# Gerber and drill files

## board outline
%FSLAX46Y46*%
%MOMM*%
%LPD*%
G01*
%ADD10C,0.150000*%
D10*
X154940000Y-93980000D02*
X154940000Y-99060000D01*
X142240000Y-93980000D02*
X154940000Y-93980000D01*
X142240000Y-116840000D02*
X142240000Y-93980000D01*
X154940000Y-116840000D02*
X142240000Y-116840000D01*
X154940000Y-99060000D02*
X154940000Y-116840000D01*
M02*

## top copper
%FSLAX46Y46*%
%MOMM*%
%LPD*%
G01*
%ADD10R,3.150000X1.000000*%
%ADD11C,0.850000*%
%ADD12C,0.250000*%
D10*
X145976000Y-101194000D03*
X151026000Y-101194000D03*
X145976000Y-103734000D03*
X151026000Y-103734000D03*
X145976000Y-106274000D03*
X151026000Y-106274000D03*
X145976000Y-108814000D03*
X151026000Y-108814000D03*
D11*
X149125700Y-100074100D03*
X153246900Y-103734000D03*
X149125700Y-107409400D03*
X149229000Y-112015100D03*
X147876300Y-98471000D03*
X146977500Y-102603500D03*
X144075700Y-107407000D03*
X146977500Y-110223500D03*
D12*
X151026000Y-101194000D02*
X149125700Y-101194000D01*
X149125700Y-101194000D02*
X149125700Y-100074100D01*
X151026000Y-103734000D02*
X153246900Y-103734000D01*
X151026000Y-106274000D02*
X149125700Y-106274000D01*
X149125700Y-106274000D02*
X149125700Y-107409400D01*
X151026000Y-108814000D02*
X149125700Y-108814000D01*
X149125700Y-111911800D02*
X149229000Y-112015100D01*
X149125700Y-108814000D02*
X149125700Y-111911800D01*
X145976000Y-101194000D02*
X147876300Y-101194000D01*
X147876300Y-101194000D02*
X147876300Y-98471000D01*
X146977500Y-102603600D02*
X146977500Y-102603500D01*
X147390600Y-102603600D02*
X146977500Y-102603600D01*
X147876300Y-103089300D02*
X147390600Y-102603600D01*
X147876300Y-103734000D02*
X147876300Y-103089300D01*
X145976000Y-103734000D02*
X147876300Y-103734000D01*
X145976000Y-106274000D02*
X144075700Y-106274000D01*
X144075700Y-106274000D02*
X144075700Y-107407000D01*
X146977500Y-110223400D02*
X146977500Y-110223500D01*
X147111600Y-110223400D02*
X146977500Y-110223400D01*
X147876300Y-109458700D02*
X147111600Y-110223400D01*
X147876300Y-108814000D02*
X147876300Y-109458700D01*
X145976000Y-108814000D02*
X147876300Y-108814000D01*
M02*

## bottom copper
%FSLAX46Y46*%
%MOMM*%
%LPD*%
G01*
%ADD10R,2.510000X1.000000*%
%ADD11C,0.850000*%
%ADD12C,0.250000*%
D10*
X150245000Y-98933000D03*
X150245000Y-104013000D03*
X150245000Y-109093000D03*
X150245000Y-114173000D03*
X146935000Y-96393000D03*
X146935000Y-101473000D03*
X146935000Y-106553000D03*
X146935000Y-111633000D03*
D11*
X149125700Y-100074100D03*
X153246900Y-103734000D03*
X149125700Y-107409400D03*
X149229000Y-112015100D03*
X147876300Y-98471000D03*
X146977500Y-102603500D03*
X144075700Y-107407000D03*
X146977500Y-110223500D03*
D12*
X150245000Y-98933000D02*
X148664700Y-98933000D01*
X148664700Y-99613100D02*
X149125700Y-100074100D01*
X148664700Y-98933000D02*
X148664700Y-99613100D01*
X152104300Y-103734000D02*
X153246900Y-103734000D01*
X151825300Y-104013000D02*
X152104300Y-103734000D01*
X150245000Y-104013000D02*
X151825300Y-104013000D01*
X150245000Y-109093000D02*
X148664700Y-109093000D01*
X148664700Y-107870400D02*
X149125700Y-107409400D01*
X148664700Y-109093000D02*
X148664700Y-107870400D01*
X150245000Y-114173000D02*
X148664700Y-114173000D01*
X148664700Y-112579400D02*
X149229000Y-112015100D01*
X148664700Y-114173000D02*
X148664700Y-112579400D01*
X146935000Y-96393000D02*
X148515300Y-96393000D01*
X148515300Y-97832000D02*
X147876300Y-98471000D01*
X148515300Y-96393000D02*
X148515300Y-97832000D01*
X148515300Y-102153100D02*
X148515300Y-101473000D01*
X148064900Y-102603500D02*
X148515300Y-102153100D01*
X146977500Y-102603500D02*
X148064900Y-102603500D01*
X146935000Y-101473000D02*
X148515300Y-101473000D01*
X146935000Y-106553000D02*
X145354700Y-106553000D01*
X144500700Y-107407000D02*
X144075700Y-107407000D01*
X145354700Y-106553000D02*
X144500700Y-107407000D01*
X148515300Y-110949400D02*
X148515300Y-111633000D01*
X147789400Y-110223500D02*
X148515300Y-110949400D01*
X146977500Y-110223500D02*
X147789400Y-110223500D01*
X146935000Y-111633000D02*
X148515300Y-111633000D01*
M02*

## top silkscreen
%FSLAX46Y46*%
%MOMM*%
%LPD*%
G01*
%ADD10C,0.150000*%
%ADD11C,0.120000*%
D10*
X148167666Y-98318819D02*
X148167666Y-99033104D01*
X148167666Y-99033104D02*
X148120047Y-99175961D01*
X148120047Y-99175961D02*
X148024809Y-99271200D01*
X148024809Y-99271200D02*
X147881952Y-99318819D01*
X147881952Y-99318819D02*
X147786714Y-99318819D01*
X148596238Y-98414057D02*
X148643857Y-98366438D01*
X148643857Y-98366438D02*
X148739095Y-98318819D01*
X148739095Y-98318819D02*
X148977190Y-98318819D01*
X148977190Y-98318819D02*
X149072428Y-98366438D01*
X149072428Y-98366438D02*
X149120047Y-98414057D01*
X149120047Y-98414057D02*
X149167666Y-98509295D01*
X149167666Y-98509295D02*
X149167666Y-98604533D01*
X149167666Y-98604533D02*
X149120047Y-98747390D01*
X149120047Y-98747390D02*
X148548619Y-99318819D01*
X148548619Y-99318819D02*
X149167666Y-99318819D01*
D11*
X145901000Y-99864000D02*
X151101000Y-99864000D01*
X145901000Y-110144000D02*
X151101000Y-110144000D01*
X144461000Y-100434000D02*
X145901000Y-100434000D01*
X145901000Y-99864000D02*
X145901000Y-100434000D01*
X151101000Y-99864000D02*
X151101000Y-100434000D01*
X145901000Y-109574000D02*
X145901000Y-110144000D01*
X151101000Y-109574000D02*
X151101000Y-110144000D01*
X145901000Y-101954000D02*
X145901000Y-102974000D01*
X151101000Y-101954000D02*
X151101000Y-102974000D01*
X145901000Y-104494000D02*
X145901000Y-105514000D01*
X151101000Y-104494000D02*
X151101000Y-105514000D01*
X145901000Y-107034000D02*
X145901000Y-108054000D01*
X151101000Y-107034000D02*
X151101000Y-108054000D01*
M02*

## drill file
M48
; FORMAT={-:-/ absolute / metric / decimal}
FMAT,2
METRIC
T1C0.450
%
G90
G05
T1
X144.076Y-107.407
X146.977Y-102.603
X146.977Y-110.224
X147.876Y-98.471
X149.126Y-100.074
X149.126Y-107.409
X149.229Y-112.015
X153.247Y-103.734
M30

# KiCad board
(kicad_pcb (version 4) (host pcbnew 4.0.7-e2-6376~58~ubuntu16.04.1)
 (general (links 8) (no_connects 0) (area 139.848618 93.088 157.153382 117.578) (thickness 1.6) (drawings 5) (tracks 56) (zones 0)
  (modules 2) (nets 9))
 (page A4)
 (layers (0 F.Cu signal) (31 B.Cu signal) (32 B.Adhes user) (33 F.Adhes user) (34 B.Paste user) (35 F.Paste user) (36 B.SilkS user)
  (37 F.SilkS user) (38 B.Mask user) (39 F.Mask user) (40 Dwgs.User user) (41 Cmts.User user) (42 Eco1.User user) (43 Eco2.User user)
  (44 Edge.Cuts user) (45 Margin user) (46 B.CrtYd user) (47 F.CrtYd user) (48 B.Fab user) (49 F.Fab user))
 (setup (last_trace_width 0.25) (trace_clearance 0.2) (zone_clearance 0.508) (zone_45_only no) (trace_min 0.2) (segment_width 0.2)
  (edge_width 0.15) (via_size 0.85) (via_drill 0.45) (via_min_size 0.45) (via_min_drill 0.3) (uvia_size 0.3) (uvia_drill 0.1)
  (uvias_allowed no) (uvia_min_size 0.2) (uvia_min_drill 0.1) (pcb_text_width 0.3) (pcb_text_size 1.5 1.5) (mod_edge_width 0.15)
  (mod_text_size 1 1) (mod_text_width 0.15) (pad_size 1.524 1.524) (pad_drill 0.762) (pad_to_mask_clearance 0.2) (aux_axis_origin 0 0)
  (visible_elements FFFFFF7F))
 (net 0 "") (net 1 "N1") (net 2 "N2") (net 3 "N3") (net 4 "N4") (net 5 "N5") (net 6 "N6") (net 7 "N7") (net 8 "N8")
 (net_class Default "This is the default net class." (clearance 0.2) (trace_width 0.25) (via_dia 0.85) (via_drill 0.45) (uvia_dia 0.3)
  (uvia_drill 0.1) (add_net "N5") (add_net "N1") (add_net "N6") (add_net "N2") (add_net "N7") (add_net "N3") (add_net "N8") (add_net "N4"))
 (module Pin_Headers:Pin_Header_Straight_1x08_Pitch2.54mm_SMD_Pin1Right (layer B.Cu) (at 148.59 105.283 180)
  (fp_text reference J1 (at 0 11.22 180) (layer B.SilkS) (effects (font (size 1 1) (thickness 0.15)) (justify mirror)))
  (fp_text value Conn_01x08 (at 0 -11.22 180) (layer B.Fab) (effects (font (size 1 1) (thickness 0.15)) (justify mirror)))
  (pad 2 smd rect (at -1.655 6.35 180) (size 2.51 1) (layers B.Cu B.Paste B.Mask) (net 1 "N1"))
  (pad 4 smd rect (at -1.655 1.27 180) (size 2.51 1) (layers B.Cu B.Paste B.Mask) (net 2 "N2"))
  (pad 6 smd rect (at -1.655 -3.81 180) (size 2.51 1) (layers B.Cu B.Paste B.Mask) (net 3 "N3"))
  (pad 8 smd rect (at -1.655 -8.89 180) (size 2.51 1) (layers B.Cu B.Paste B.Mask) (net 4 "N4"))
  (pad 1 smd rect (at 1.655 8.89 180) (size 2.51 1) (layers B.Cu B.Paste B.Mask) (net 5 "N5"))
  (pad 3 smd rect (at 1.655 3.81 180) (size 2.51 1) (layers B.Cu B.Paste B.Mask) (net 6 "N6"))
  (pad 5 smd rect (at 1.655 -1.27 180) (size 2.51 1) (layers B.Cu B.Paste B.Mask) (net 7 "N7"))
  (pad 7 smd rect (at 1.655 -6.35 180) (size 2.51 1) (layers B.Cu B.Paste B.Mask) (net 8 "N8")))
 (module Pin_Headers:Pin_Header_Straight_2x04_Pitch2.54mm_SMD (layer F.Cu) (at 148.501 105.004)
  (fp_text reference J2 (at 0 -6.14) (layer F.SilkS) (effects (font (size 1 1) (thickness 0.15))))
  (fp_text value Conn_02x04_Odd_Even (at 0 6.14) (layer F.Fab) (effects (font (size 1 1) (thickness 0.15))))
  (fp_line (start -2.6 -5.14) (end 2.6 -5.14) (layer F.SilkS) (width 0.12))
  (fp_line (start -2.6 5.14) (end 2.6 5.14) (layer F.SilkS) (width 0.12))
  (fp_line (start -4.04 -4.57) (end -2.6 -4.57) (layer F.SilkS) (width 0.12))
  (fp_line (start -2.6 -5.14) (end -2.6 -4.57) (layer F.SilkS) (width 0.12))
  (fp_line (start 2.6 -5.14) (end 2.6 -4.57) (layer F.SilkS) (width 0.12))
  (fp_line (start -2.6 4.57) (end -2.6 5.14) (layer F.SilkS) (width 0.12))
  (fp_line (start 2.6 4.57) (end 2.6 5.14) (layer F.SilkS) (width 0.12))
  (fp_line (start -2.6 -3.05) (end -2.6 -2.03) (layer F.SilkS) (width 0.12))
  (fp_line (start 2.6 -3.05) (end 2.6 -2.03) (layer F.SilkS) (width 0.12))
  (fp_line (start -2.6 -0.51) (end -2.6 0.51) (layer F.SilkS) (width 0.12))
  (fp_line (start 2.6 -0.51) (end 2.6 0.51) (layer F.SilkS) (width 0.12))
  (fp_line (start -2.6 2.03) (end -2.6 3.05) (layer F.SilkS) (width 0.12))
  (fp_line (start 2.6 2.03) (end 2.6 3.05) (layer F.SilkS) (width 0.12))
  (pad 1 smd rect (at -2.525 -3.81) (size 3.15 1) (layers F.Cu F.Paste F.Mask) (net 5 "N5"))
  (pad 2 smd rect (at 2.525 -3.81) (size 3.15 1) (layers F.Cu F.Paste F.Mask) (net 1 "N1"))
  (pad 3 smd rect (at -2.525 -1.27) (size 3.15 1) (layers F.Cu F.Paste F.Mask) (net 6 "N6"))
  (pad 4 smd rect (at 2.525 -1.27) (size 3.15 1) (layers F.Cu F.Paste F.Mask) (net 2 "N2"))
  (pad 5 smd rect (at -2.525 1.27) (size 3.15 1) (layers F.Cu F.Paste F.Mask) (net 7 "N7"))
  (pad 6 smd rect (at 2.525 1.27) (size 3.15 1) (layers F.Cu F.Paste F.Mask) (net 3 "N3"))
  (pad 7 smd rect (at -2.525 3.81) (size 3.15 1) (layers F.Cu F.Paste F.Mask) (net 8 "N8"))
  (pad 8 smd rect (at 2.525 3.81) (size 3.15 1) (layers F.Cu F.Paste F.Mask) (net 4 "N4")))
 (gr_line (start 154.94 93.98) (end 154.94 99.06) (layer Edge.Cuts) (width 0.15))
 (gr_line (start 142.24 93.98) (end 154.94 93.98) (layer Edge.Cuts) (width 0.15))
 (gr_line (start 142.24 116.84) (end 142.24 93.98) (layer Edge.Cuts) (width 0.15))
 (gr_line (start 154.94 116.84) (end 142.24 116.84) (layer Edge.Cuts) (width 0.15))
 (gr_line (start 154.94 99.06) (end 154.94 116.84) (layer Edge.Cuts) (width 0.15))
 (via (at 149.1257 100.0741) (size 0.85) (layers F.Cu B.Cu) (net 1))
 (segment (start 151.026 101.194) (end 149.1257 101.194) (width 0.25) (layer F.Cu) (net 1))
 (segment (start 150.245 98.933) (end 148.6647 98.933) (width 0.25) (layer B.Cu) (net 1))
 (segment (start 148.6647 99.6131) (end 149.1257 100.0741) (width 0.25) (layer B.Cu) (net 1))
 (segment (start 148.6647 98.933) (end 148.6647 99.6131) (width 0.25) (layer B.Cu) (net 1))
 (segment (start 149.1257 101.194) (end 149.1257 100.0741) (width 0.25) (layer F.Cu) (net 1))
 (via (at 153.2469 103.734) (size 0.85) (layers F.Cu B.Cu) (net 2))
 (segment (start 152.1043 103.734) (end 153.2469 103.734) (width 0.25) (layer B.Cu) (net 2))
 (segment (start 151.8253 104.013) (end 152.1043 103.734) (width 0.25) (layer B.Cu) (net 2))
 (segment (start 151.026 103.734) (end 153.2469 103.734) (width 0.25) (layer F.Cu) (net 2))
 (segment (start 150.245 104.013) (end 151.8253 104.013) (width 0.25) (layer B.Cu) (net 2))
 (via (at 149.1257 107.4094) (size 0.85) (layers F.Cu B.Cu) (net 3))
 (segment (start 151.026 106.274) (end 149.1257 106.274) (width 0.25) (layer F.Cu) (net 3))
 (segment (start 150.245 109.093) (end 148.6647 109.093) (width 0.25) (layer B.Cu) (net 3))
 (segment (start 148.6647 107.8704) (end 149.1257 107.4094) (width 0.25) (layer B.Cu) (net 3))
 (segment (start 148.6647 109.093) (end 148.6647 107.8704) (width 0.25) (layer B.Cu) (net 3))
 (segment (start 149.1257 106.274) (end 149.1257 107.4094) (width 0.25) (layer F.Cu) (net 3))
 (via (at 149.229 112.0151) (size 0.85) (layers F.Cu B.Cu) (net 4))
 (segment (start 150.245 114.173) (end 148.6647 114.173) (width 0.25) (layer B.Cu) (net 4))
 (segment (start 151.026 108.814) (end 149.1257 108.814) (width 0.25) (layer F.Cu) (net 4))
 (segment (start 148.6647 112.5794) (end 149.229 112.0151) (width 0.25) (layer B.Cu) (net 4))
 (segment (start 148.6647 114.173) (end 148.6647 112.5794) (width 0.25) (layer B.Cu) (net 4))
 (segment (start 149.1257 111.9118) (end 149.229 112.0151) (width 0.25) (layer F.Cu) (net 4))
 (segment (start 149.1257 108.814) (end 149.1257 111.9118) (width 0.25) (layer F.Cu) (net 4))
 (via (at 147.8763 98.471) (size 0.85) (layers F.Cu B.Cu) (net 5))
 (segment (start 146.935 96.393) (end 148.5153 96.393) (width 0.25) (layer B.Cu) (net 5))
 (segment (start 145.976 101.194) (end 147.8763 101.194) (width 0.25) (layer F.Cu) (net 5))
 (segment (start 148.5153 97.832) (end 147.8763 98.471) (width 0.25) (layer B.Cu) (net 5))
 (segment (start 148.5153 96.393) (end 148.5153 97.832) (width 0.25) (layer B.Cu) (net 5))
 (segment (start 147.8763 101.194) (end 147.8763 98.471) (width 0.25) (layer F.Cu) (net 5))
 (via (at 146.9775 102.6035) (size 0.85) (layers F.Cu B.Cu) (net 6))
 (segment (start 146.9775 102.6036) (end 146.9775 102.6035) (width 0.25) (layer F.Cu) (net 6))
 (segment (start 147.3906 102.6036) (end 146.9775 102.6036) (width 0.25) (layer F.Cu) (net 6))
 (segment (start 147.8763 103.0893) (end 147.3906 102.6036) (width 0.25) (layer F.Cu) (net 6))
 (segment (start 147.8763 103.734) (end 147.8763 103.0893) (width 0.25) (layer F.Cu) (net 6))
 (segment (start 148.5153 102.1531) (end 148.5153 101.473) (width 0.25) (layer B.Cu) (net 6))
 (segment (start 148.0649 102.6035) (end 148.5153 102.1531) (width 0.25) (layer B.Cu) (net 6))
 (segment (start 146.9775 102.6035) (end 148.0649 102.6035) (width 0.25) (layer B.Cu) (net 6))
 (segment (start 145.976 103.734) (end 147.8763 103.734) (width 0.25) (layer F.Cu) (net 6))
 (segment (start 146.935 101.473) (end 148.5153 101.473) (width 0.25) (layer B.Cu) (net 6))
 (via (at 144.0757 107.407) (size 0.85) (layers F.Cu B.Cu) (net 7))
 (segment (start 145.976 106.274) (end 144.0757 106.274) (width 0.25) (layer F.Cu) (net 7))
 (segment (start 146.935 106.553) (end 145.3547 106.553) (width 0.25) (layer B.Cu) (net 7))
 (segment (start 144.5007 107.407) (end 144.0757 107.407) (width 0.25) (layer B.Cu) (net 7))
 (segment (start 145.3547 106.553) (end 144.5007 107.407) (width 0.25) (layer B.Cu) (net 7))
 (segment (start 144.0757 106.274) (end 144.0757 107.407) (width 0.25) (layer F.Cu) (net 7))
 (via (at 146.9775 110.2235) (size 0.85) (layers F.Cu B.Cu) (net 8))
 (segment (start 146.9775 110.2234) (end 146.9775 110.2235) (width 0.25) (layer F.Cu) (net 8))
 (segment (start 147.1116 110.2234) (end 146.9775 110.2234) (width 0.25) (layer F.Cu) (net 8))
 (segment (start 147.8763 109.4587) (end 147.1116 110.2234) (width 0.25) (layer F.Cu) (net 8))
 (segment (start 147.8763 108.814) (end 147.8763 109.4587) (width 0.25) (layer F.Cu) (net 8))
 (segment (start 148.5153 110.9494) (end 148.5153 111.633) (width 0.25) (layer B.Cu) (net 8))
 (segment (start 147.7894 110.2235) (end 148.5153 110.9494) (width 0.25) (layer B.Cu) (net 8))
 (segment (start 146.9775 110.2235) (end 147.7894 110.2235) (width 0.25) (layer B.Cu) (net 8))
 (segment (start 145.976 108.814) (end 147.8763 108.814) (width 0.25) (layer F.Cu) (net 8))
 (segment (start 146.935 111.633) (end 148.5153 111.633) (width 0.25) (layer B.Cu) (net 8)))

